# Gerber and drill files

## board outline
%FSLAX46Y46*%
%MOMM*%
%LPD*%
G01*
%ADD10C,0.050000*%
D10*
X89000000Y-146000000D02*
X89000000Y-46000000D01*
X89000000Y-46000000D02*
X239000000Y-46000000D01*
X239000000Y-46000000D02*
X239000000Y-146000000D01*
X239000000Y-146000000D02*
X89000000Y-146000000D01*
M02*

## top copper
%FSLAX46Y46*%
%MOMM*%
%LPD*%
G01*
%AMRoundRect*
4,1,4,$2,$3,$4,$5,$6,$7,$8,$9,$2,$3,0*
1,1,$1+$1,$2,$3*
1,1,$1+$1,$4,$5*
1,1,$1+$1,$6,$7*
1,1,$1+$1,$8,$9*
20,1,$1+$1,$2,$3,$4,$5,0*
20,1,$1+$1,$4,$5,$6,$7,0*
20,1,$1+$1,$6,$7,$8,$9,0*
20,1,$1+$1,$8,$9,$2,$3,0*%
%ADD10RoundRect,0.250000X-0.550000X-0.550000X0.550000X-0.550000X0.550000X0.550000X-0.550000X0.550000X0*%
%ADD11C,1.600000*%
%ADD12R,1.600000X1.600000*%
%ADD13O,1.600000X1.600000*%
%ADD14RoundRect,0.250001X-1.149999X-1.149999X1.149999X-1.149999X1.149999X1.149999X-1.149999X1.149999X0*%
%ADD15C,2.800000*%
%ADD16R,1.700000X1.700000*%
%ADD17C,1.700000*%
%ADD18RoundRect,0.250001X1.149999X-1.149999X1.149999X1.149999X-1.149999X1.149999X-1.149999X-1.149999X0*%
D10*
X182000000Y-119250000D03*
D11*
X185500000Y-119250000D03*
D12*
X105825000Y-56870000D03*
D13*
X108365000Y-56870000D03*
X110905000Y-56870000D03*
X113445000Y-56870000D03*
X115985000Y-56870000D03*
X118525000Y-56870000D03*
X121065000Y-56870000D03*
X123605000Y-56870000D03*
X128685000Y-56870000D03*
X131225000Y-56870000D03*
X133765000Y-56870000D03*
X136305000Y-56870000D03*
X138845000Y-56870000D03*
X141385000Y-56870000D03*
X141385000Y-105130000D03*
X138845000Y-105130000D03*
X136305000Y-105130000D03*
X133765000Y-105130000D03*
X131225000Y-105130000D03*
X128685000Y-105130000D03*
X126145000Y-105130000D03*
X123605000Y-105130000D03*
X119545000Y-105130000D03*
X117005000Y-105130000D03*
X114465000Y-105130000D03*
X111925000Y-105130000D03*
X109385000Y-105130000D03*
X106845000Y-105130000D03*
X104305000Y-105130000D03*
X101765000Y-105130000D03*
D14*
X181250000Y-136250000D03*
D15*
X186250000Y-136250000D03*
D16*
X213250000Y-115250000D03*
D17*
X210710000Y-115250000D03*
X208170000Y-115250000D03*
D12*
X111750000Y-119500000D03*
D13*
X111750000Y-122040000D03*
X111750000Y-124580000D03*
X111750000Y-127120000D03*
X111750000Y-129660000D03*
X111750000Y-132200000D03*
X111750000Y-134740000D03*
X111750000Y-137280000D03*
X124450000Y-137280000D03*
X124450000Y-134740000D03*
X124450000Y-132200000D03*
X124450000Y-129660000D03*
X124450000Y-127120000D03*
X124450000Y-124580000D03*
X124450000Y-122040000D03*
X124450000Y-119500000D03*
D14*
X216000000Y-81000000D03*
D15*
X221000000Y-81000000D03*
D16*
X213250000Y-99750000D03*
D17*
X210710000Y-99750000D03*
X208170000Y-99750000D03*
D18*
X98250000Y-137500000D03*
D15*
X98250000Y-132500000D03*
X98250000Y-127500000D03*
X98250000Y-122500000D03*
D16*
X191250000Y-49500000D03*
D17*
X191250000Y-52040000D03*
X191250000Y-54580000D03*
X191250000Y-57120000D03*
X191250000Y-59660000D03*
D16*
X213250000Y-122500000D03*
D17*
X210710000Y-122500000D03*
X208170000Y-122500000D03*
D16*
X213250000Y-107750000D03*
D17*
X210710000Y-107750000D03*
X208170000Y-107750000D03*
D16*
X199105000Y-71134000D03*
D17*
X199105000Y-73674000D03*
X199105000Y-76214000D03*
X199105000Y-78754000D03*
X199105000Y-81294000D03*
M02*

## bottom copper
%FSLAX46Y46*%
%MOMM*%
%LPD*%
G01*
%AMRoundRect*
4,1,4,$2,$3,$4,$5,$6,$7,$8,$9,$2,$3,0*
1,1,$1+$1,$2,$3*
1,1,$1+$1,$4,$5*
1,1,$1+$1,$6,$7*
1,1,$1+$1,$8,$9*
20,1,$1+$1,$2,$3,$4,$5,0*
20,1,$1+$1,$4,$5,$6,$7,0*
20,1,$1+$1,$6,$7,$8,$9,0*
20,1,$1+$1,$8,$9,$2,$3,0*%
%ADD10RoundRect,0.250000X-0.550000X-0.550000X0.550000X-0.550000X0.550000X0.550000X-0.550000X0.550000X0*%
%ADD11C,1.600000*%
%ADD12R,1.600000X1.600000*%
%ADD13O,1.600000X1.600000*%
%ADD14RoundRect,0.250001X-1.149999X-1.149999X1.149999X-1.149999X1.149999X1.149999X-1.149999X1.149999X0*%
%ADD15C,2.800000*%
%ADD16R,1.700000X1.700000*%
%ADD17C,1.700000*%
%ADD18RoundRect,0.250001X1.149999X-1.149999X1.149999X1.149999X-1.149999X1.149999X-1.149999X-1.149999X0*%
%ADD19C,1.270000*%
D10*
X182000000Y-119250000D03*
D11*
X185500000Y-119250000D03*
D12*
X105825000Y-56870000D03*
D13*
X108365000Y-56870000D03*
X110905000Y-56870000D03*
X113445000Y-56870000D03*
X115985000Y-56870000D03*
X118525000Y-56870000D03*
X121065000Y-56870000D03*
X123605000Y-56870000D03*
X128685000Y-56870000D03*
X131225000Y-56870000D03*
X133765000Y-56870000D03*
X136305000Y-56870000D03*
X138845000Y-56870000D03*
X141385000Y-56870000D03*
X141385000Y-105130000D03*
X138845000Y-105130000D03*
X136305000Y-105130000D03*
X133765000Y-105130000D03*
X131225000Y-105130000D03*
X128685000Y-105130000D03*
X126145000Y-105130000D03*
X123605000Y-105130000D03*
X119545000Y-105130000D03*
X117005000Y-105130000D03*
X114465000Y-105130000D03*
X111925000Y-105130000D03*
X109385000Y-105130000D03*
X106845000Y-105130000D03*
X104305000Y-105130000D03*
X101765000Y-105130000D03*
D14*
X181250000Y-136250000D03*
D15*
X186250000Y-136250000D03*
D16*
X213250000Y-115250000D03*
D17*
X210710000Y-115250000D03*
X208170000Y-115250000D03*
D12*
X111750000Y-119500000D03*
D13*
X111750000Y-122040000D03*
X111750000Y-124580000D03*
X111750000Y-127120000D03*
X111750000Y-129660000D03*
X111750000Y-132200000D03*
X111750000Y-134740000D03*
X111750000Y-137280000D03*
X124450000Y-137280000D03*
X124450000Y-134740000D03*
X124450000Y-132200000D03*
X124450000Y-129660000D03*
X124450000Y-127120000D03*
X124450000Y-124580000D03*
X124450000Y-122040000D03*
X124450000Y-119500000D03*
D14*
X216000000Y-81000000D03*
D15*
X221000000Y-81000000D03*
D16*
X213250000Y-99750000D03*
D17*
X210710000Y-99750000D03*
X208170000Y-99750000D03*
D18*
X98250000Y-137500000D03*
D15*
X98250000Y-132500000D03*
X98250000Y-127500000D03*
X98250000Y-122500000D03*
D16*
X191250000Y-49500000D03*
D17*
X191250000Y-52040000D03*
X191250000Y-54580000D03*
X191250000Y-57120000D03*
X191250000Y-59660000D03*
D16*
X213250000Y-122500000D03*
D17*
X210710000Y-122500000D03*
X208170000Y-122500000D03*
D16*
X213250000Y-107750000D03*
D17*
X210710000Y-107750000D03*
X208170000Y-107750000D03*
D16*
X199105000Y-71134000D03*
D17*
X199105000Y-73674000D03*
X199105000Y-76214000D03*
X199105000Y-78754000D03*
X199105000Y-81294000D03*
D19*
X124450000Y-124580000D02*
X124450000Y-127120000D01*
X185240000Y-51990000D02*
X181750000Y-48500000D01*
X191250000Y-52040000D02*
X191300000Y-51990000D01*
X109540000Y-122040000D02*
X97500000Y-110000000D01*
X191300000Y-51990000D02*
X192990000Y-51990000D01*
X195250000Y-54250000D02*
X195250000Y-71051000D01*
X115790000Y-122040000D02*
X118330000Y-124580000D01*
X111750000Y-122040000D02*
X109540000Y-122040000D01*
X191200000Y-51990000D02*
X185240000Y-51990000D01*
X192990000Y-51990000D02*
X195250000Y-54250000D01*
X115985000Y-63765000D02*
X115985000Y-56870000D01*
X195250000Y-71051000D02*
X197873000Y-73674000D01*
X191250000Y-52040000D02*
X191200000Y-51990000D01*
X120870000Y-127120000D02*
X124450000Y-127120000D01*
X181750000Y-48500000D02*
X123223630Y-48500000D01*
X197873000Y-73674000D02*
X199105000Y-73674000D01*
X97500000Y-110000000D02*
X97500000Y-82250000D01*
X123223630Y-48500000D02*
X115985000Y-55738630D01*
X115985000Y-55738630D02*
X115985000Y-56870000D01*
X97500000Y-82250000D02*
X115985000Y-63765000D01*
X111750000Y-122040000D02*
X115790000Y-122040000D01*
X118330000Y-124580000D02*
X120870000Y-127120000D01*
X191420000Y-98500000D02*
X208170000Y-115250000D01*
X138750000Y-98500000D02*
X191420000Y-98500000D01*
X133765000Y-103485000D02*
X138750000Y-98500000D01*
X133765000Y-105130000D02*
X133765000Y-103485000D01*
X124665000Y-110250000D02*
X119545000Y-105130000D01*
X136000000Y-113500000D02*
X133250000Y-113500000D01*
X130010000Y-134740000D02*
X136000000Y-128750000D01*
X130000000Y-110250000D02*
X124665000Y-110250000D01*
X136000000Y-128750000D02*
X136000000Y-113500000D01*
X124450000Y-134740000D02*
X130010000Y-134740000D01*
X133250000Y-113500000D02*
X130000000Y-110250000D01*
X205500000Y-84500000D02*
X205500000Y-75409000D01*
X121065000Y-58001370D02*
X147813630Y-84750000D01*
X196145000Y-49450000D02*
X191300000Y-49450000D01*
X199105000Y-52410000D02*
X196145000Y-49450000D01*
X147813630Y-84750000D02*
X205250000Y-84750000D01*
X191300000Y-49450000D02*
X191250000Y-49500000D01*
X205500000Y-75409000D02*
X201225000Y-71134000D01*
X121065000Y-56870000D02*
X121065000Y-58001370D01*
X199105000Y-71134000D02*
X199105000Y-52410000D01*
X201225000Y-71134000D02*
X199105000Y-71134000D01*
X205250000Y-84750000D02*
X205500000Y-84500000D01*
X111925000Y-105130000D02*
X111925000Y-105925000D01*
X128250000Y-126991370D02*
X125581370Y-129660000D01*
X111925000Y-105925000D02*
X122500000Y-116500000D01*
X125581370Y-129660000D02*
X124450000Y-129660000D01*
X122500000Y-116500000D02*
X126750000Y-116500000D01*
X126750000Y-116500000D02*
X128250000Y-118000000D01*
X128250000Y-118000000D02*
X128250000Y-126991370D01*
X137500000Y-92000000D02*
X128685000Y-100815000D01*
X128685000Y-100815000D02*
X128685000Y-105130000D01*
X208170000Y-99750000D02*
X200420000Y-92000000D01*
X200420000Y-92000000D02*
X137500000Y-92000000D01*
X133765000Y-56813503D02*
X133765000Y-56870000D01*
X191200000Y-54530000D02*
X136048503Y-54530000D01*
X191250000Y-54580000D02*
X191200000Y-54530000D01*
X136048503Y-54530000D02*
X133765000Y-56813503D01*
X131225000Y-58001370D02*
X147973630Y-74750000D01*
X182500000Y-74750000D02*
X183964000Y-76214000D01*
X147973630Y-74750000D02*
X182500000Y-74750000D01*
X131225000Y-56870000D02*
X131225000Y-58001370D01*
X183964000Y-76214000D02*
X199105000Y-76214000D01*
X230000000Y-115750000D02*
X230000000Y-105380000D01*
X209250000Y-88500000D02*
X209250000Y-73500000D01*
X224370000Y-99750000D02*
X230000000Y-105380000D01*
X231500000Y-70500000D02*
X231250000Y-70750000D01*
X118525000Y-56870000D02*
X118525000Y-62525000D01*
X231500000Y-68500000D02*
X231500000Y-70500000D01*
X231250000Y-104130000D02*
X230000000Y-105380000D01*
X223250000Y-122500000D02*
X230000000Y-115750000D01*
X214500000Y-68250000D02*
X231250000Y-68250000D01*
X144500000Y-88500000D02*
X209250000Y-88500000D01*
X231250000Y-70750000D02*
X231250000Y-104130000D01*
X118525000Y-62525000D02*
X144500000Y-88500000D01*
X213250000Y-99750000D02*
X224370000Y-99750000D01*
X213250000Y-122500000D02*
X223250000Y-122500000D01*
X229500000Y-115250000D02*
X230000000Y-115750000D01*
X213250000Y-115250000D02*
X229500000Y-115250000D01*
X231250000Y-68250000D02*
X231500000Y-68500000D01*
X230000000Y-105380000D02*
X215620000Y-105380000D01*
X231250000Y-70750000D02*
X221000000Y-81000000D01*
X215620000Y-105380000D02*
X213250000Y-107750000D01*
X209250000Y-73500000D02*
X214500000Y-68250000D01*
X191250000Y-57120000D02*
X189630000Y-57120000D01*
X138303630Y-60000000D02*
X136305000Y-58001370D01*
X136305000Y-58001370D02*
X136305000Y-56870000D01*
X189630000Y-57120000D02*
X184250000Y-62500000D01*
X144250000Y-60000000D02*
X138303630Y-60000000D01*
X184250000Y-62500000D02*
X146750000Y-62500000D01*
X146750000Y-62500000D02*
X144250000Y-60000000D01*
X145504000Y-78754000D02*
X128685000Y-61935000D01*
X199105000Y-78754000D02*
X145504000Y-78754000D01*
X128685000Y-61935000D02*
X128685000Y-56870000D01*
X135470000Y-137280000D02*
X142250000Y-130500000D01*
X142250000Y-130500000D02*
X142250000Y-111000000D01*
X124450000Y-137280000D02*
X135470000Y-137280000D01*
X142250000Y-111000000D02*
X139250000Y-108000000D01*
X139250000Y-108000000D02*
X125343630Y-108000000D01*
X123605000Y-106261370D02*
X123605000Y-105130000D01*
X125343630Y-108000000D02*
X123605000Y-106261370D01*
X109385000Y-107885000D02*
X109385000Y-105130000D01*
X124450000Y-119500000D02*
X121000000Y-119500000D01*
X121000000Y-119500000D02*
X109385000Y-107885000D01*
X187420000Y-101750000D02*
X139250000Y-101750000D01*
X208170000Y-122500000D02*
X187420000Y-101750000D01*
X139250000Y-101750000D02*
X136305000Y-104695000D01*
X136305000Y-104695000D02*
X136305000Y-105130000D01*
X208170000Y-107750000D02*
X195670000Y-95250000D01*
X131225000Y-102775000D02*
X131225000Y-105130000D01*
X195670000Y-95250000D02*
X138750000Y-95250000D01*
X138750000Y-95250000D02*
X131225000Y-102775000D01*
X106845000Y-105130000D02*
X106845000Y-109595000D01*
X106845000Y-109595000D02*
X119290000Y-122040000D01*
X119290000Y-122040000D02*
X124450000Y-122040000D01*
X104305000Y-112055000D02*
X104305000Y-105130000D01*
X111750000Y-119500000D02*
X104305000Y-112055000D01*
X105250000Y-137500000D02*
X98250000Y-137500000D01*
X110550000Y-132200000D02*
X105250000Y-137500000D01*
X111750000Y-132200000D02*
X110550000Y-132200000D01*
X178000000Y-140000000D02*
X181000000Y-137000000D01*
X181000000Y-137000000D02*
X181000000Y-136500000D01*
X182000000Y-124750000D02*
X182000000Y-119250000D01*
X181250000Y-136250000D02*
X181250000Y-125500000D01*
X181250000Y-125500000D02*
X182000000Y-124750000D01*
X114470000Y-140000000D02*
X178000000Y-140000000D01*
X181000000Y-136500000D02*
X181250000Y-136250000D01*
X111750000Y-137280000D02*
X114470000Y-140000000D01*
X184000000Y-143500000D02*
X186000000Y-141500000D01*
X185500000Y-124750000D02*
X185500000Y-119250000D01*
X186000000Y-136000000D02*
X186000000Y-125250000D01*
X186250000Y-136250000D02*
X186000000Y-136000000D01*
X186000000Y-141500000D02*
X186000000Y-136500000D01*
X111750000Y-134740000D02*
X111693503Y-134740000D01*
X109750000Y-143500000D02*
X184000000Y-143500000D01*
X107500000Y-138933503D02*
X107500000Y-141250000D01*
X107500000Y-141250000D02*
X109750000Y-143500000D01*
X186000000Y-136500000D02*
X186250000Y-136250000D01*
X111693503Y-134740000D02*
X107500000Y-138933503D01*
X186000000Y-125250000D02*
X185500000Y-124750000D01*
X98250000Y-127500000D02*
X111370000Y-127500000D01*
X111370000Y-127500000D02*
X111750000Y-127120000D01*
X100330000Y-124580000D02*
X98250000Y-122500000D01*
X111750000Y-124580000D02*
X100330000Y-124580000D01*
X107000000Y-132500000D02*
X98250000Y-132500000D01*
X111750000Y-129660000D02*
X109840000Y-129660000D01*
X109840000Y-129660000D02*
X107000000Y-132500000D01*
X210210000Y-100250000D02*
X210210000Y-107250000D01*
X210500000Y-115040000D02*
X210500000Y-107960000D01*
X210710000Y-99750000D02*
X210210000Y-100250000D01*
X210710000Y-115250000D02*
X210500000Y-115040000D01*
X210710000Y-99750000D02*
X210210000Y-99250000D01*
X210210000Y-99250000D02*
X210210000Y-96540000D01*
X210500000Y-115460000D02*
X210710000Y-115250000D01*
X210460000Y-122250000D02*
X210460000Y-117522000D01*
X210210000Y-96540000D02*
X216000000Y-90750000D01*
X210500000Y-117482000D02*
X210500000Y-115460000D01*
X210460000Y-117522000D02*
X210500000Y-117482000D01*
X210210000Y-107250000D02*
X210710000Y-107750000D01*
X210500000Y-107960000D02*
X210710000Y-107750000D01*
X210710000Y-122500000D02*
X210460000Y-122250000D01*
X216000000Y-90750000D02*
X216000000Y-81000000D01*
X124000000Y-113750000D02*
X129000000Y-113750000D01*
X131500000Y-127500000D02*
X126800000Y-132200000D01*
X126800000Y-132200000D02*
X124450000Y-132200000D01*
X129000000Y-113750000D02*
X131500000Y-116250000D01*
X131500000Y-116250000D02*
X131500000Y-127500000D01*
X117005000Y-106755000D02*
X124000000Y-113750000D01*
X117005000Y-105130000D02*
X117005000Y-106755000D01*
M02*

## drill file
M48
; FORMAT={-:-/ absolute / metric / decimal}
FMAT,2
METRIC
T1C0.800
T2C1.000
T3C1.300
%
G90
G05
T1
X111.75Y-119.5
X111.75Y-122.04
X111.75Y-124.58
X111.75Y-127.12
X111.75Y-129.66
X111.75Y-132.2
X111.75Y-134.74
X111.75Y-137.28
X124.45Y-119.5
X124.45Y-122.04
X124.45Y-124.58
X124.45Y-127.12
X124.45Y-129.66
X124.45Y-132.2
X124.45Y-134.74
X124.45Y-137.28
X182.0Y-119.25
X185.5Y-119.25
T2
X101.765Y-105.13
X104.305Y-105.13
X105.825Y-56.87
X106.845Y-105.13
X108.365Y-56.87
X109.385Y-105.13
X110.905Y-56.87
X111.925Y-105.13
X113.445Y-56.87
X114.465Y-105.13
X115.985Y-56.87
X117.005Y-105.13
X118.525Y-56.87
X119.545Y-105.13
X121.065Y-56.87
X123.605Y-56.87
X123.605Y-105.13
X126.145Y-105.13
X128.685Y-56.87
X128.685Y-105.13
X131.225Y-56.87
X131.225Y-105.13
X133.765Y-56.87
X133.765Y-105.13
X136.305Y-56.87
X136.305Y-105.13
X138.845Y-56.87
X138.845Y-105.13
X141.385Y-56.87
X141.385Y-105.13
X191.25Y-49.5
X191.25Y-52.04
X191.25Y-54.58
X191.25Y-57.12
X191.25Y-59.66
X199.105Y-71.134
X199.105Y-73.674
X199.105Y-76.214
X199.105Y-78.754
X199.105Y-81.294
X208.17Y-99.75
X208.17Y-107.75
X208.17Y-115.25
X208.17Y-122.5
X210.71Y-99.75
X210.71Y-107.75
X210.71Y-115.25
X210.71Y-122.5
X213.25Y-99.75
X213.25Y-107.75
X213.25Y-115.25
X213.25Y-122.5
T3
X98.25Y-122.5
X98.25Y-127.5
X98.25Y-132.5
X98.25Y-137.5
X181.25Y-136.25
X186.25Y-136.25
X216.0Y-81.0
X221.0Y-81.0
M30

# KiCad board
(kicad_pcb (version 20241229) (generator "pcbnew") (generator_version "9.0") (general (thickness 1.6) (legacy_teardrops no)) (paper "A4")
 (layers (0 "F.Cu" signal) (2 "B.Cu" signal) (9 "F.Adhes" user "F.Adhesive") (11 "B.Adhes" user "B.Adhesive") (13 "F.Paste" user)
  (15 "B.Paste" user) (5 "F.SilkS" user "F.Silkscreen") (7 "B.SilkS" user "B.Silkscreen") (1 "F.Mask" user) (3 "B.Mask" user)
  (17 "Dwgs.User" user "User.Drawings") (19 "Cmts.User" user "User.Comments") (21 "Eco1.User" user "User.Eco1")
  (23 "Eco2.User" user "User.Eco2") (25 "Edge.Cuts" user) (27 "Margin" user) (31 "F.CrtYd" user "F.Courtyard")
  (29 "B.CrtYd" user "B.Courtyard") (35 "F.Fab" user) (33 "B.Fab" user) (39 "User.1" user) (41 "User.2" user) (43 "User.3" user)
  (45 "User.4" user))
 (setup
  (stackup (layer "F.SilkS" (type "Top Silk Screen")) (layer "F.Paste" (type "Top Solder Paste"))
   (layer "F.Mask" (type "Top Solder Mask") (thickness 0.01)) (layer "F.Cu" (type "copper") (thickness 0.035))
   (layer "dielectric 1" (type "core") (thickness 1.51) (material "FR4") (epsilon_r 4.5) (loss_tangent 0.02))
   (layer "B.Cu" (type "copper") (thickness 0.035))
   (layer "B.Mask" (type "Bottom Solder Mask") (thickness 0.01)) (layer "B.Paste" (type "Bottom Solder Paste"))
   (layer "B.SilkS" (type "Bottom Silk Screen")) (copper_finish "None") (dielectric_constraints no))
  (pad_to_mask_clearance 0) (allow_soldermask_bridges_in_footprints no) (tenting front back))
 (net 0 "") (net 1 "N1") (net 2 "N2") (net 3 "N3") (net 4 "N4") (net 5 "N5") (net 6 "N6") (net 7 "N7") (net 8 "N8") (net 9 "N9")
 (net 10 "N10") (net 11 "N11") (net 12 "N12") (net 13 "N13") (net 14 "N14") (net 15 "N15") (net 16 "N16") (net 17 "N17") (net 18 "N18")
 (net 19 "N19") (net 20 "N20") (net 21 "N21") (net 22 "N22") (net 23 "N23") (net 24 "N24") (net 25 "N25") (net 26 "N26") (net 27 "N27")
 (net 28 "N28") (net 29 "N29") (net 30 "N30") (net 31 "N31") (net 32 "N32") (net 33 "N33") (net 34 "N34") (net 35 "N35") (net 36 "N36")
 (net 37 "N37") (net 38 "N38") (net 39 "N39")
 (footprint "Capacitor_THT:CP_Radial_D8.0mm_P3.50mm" (layer "F.Cu") (at 182 119.25)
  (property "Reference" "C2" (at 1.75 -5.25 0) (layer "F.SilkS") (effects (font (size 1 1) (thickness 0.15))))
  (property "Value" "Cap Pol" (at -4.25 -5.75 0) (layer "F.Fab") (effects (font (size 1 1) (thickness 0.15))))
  (pad "1" thru_hole roundrect (at 0 0) (size 1.6 1.6) (drill 0.8) (layers "*.Cu" "*.Mask") (remove_unused_layers no)
   (roundrect_rratio 0.15625) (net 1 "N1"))
  (pad "2" thru_hole circle (at 3.5 0) (size 1.6 1.6) (drill 0.8) (layers "*.Cu" "*.Mask") (remove_unused_layers no) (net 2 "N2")))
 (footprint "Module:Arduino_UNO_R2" (layer "F.Cu") (at 105.825 56.87)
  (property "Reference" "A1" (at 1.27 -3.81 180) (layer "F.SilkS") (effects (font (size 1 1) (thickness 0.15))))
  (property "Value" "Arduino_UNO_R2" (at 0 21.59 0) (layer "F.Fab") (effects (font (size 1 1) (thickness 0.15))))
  (pad "1" thru_hole rect (at 0 0 90) (size 1.6 1.6) (drill 1) (layers "*.Cu" "*.Mask") (remove_unused_layers no) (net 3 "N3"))
  (pad "2" thru_hole oval (at 2.54 0 90) (size 1.6 1.6) (drill 1) (layers "*.Cu" "*.Mask") (remove_unused_layers no) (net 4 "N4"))
  (pad "3" thru_hole oval (at 5.08 0 90) (size 1.6 1.6) (drill 1) (layers "*.Cu" "*.Mask") (remove_unused_layers no) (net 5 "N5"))
  (pad "4" thru_hole oval (at 7.62 0 90) (size 1.6 1.6) (drill 1) (layers "*.Cu" "*.Mask") (remove_unused_layers no) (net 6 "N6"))
  (pad "5" thru_hole oval (at 10.16 0 90) (size 1.6 1.6) (drill 1) (layers "*.Cu" "*.Mask") (remove_unused_layers no) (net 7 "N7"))
  (pad "6" thru_hole oval (at 12.7 0 90) (size 1.6 1.6) (drill 1) (layers "*.Cu" "*.Mask") (remove_unused_layers no) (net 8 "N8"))
  (pad "7" thru_hole oval (at 15.24 0 90) (size 1.6 1.6) (drill 1) (layers "*.Cu" "*.Mask") (remove_unused_layers no) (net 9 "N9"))
  (pad "8" thru_hole oval (at 17.78 0 90) (size 1.6 1.6) (drill 1) (layers "*.Cu" "*.Mask") (remove_unused_layers no) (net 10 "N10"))
  (pad "9" thru_hole oval (at 22.86 0 90) (size 1.6 1.6) (drill 1) (layers "*.Cu" "*.Mask") (remove_unused_layers no) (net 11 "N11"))
  (pad "10" thru_hole oval (at 25.4 0 90) (size 1.6 1.6) (drill 1) (layers "*.Cu" "*.Mask") (remove_unused_layers no) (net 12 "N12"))
  (pad "11" thru_hole oval (at 27.94 0 90) (size 1.6 1.6) (drill 1) (layers "*.Cu" "*.Mask") (remove_unused_layers no) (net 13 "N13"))
  (pad "12" thru_hole oval (at 30.48 0 90) (size 1.6 1.6) (drill 1) (layers "*.Cu" "*.Mask") (remove_unused_layers no) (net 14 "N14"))
  (pad "13" thru_hole oval (at 33.02 0 90) (size 1.6 1.6) (drill 1) (layers "*.Cu" "*.Mask") (remove_unused_layers no) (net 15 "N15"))
  (pad "14" thru_hole oval (at 35.56 0 90) (size 1.6 1.6) (drill 1) (layers "*.Cu" "*.Mask") (remove_unused_layers no) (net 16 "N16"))
  (pad "15" thru_hole oval (at 35.56 48.26 90) (size 1.6 1.6) (drill 1) (layers "*.Cu" "*.Mask") (remove_unused_layers no) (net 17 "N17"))
  (pad "16" thru_hole oval (at 33.02 48.26 90) (size 1.6 1.6) (drill 1) (layers "*.Cu" "*.Mask") (remove_unused_layers no) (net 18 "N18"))
  (pad "17" thru_hole oval (at 30.48 48.26 90) (size 1.6 1.6) (drill 1) (layers "*.Cu" "*.Mask") (remove_unused_layers no) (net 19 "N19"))
  (pad "18" thru_hole oval (at 27.94 48.26 90) (size 1.6 1.6) (drill 1) (layers "*.Cu" "*.Mask") (remove_unused_layers no) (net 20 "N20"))
  (pad "19" thru_hole oval (at 25.4 48.26 90) (size 1.6 1.6) (drill 1) (layers "*.Cu" "*.Mask") (remove_unused_layers no) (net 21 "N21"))
  (pad "20" thru_hole oval (at 22.86 48.26 90) (size 1.6 1.6) (drill 1) (layers "*.Cu" "*.Mask") (remove_unused_layers no) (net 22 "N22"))
  (pad "21" thru_hole oval (at 20.32 48.26 90) (size 1.6 1.6) (drill 1) (layers "*.Cu" "*.Mask") (remove_unused_layers no) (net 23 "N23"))
  (pad "22" thru_hole oval (at 17.78 48.26 90) (size 1.6 1.6) (drill 1) (layers "*.Cu" "*.Mask") (remove_unused_layers no) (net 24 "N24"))
  (pad "23" thru_hole oval (at 13.72 48.26 90) (size 1.6 1.6) (drill 1) (layers "*.Cu" "*.Mask") (remove_unused_layers no) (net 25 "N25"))
  (pad "24" thru_hole oval (at 11.18 48.26 90) (size 1.6 1.6) (drill 1) (layers "*.Cu" "*.Mask") (remove_unused_layers no) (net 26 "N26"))
  (pad "25" thru_hole oval (at 8.64 48.26 90) (size 1.6 1.6) (drill 1) (layers "*.Cu" "*.Mask") (remove_unused_layers no) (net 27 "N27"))
  (pad "26" thru_hole oval (at 6.1 48.26 90) (size 1.6 1.6) (drill 1) (layers "*.Cu" "*.Mask") (remove_unused_layers no) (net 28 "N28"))
  (pad "27" thru_hole oval (at 3.56 48.26 90) (size 1.6 1.6) (drill 1) (layers "*.Cu" "*.Mask") (remove_unused_layers no) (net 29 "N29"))
  (pad "28" thru_hole oval (at 1.02 48.26 90) (size 1.6 1.6) (drill 1) (layers "*.Cu" "*.Mask") (remove_unused_layers no) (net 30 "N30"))
  (pad "29" thru_hole oval (at -1.52 48.26 90) (size 1.6 1.6) (drill 1) (layers "*.Cu" "*.Mask") (remove_unused_layers no) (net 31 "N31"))
  (pad "30" thru_hole oval (at -4.06 48.26 90) (size 1.6 1.6) (drill 1) (layers "*.Cu" "*.Mask") (remove_unused_layers no) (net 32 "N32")))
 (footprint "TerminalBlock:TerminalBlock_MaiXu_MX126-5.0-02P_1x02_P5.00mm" (layer "F.Cu") (at 181.25 136.25)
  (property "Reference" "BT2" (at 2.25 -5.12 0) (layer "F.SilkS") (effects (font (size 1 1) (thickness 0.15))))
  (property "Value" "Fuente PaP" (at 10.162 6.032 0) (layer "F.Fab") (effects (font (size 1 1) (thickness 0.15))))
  (pad "1" thru_hole roundrect (at 0 0) (size 2.8 2.8) (drill 1.3) (layers "*.Cu" "*.Mask") (remove_unused_layers no)
   (roundrect_rratio 0.089286) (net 1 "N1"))
  (pad "2" thru_hole circle (at 5 0) (size 2.8 2.8) (drill 1.3) (layers "*.Cu" "*.Mask") (remove_unused_layers no) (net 2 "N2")))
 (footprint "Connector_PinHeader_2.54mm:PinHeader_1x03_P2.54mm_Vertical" (layer "F.Cu") (at 213.25 115.25 -90)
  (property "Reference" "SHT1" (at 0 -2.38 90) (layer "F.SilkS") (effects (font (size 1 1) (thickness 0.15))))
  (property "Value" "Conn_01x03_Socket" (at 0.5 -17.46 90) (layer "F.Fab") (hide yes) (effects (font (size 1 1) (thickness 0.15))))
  (pad "1" thru_hole rect (at 0 0 270) (size 1.7 1.7) (drill 1) (layers "*.Cu" "*.Mask") (remove_unused_layers no) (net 8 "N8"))
  (pad "2" thru_hole circle (at 0 2.54 270) (size 1.7 1.7) (drill 1) (layers "*.Cu" "*.Mask") (remove_unused_layers no) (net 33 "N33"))
  (pad "3" thru_hole circle (at 0 5.08 270) (size 1.7 1.7) (drill 1) (layers "*.Cu" "*.Mask") (remove_unused_layers no) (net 20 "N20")))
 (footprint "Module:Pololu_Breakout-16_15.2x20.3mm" (layer "F.Cu") (at 111.75 119.5)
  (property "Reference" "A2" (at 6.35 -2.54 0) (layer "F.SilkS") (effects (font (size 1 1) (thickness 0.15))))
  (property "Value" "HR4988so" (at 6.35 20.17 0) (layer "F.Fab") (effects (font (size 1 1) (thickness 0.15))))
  (pad "1" thru_hole rect (at 0 0) (size 1.6 1.6) (drill 0.8) (layers "*.Cu" "*.Mask") (remove_unused_layers no) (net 31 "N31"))
  (pad "2" thru_hole oval (at 0 2.54) (size 1.6 1.6) (drill 0.8) (layers "*.Cu" "*.Mask") (remove_unused_layers no) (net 7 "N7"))
  (pad "3" thru_hole oval (at 0 5.08) (size 1.6 1.6) (drill 0.8) (layers "*.Cu" "*.Mask") (remove_unused_layers no) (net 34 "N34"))
  (pad "4" thru_hole oval (at 0 7.62) (size 1.6 1.6) (drill 0.8) (layers "*.Cu" "*.Mask") (remove_unused_layers no) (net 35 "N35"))
  (pad "5" thru_hole oval (at 0 10.16) (size 1.6 1.6) (drill 0.8) (layers "*.Cu" "*.Mask") (remove_unused_layers no) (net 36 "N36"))
  (pad "6" thru_hole oval (at 0 12.7) (size 1.6 1.6) (drill 0.8) (layers "*.Cu" "*.Mask") (remove_unused_layers no) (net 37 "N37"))
  (pad "7" thru_hole oval (at 0 15.24) (size 1.6 1.6) (drill 0.8) (layers "*.Cu" "*.Mask") (remove_unused_layers no) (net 2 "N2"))
  (pad "8" thru_hole oval (at 0 17.78) (size 1.6 1.6) (drill 0.8) (layers "*.Cu" "*.Mask") (remove_unused_layers no) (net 1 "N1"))
  (pad "9" thru_hole oval (at 12.7 17.78) (size 1.6 1.6) (drill 0.8) (layers "*.Cu" "*.Mask") (remove_unused_layers no) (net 24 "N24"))
  (pad "10" thru_hole oval (at 12.7 15.24) (size 1.6 1.6) (drill 0.8) (layers "*.Cu" "*.Mask") (remove_unused_layers no) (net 25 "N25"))
  (pad "11" thru_hole oval (at 12.7 12.7) (size 1.6 1.6) (drill 0.8) (layers "*.Cu" "*.Mask") (remove_unused_layers no) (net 26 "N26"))
  (pad "12" thru_hole oval (at 12.7 10.16) (size 1.6 1.6) (drill 0.8) (layers "*.Cu" "*.Mask") (remove_unused_layers no) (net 28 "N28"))
  (pad "13" thru_hole oval (at 12.7 7.62) (size 1.6 1.6) (drill 0.8) (layers "*.Cu" "*.Mask") (remove_unused_layers no) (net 7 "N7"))
  (pad "14" thru_hole oval (at 12.7 5.08) (size 1.6 1.6) (drill 0.8) (layers "*.Cu" "*.Mask") (remove_unused_layers no) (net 7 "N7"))
  (pad "15" thru_hole oval (at 12.7 2.54) (size 1.6 1.6) (drill 0.8) (layers "*.Cu" "*.Mask") (remove_unused_layers no) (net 30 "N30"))
  (pad "16" thru_hole oval (at 12.7 0) (size 1.6 1.6) (drill 0.8) (layers "*.Cu" "*.Mask") (remove_unused_layers no) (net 29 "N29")))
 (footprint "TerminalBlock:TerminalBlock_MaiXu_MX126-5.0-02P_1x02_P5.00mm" (layer "F.Cu") (at 216 81)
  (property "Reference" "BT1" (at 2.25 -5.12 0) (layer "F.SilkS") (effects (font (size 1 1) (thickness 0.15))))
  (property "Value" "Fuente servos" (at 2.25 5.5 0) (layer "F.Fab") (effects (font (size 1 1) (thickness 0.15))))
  (pad "1" thru_hole roundrect (at 0 0) (size 2.8 2.8) (drill 1.3) (layers "*.Cu" "*.Mask") (remove_unused_layers no)
   (roundrect_rratio 0.089286) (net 33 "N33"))
  (pad "2" thru_hole circle (at 5 0) (size 2.8 2.8) (drill 1.3) (layers "*.Cu" "*.Mask") (remove_unused_layers no) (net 8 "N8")))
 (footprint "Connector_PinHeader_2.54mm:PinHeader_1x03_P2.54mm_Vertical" (layer "F.Cu") (at 213.25 99.75 -90)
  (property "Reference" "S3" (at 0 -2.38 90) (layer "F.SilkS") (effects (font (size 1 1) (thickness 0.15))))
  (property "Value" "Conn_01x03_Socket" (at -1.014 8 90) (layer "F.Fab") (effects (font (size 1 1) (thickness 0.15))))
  (pad "1" thru_hole rect (at 0 0 270) (size 1.7 1.7) (drill 1) (layers "*.Cu" "*.Mask") (remove_unused_layers no) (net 8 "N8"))
  (pad "2" thru_hole circle (at 0 2.54 270) (size 1.7 1.7) (drill 1) (layers "*.Cu" "*.Mask") (remove_unused_layers no) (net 33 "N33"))
  (pad "3" thru_hole circle (at 0 5.08 270) (size 1.7 1.7) (drill 1) (layers "*.Cu" "*.Mask") (remove_unused_layers no) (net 22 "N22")))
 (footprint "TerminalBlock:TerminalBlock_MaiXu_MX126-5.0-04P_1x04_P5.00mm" (layer "F.Cu") (at 98.25 137.5 90)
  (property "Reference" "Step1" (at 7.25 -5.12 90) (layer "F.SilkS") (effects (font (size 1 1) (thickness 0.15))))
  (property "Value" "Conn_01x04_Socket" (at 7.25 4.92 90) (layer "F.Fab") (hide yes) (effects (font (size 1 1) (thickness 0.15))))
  (pad "1" thru_hole roundrect (at 0 0 90) (size 2.8 2.8) (drill 1.3) (layers "*.Cu" "*.Mask") (remove_unused_layers no)
   (roundrect_rratio 0.089286) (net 37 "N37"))
  (pad "2" thru_hole circle (at 5 0 90) (size 2.8 2.8) (drill 1.3) (layers "*.Cu" "*.Mask") (remove_unused_layers no) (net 36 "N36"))
  (pad "3" thru_hole circle (at 10 0 90) (size 2.8 2.8) (drill 1.3) (layers "*.Cu" "*.Mask") (remove_unused_layers no) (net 35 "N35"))
  (pad "4" thru_hole circle (at 15 0 90) (size 2.8 2.8) (drill 1.3) (layers "*.Cu" "*.Mask") (remove_unused_layers no) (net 34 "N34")))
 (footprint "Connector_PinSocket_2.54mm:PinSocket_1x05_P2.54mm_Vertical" (layer "F.Cu") (at 191.25 49.5)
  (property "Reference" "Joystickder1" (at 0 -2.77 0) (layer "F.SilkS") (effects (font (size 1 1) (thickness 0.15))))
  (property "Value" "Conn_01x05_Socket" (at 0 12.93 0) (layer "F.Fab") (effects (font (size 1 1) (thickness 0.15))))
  (pad "1" thru_hole rect (at 0 0) (size 1.7 1.7) (drill 1) (layers "*.Cu" "*.Mask") (remove_unused_layers no) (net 9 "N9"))
  (pad "2" thru_hole circle (at 0 2.54) (size 1.7 1.7) (drill 1) (layers "*.Cu" "*.Mask") (remove_unused_layers no) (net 7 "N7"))
  (pad "3" thru_hole circle (at 0 5.08) (size 1.7 1.7) (drill 1) (layers "*.Cu" "*.Mask") (remove_unused_layers no) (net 13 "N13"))
  (pad "4" thru_hole circle (at 0 7.62) (size 1.7 1.7) (drill 1) (layers "*.Cu" "*.Mask") (remove_unused_layers no) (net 14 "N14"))
  (pad "5" thru_hole circle (at 0 10.16) (size 1.7 1.7) (drill 1) (layers "*.Cu" "*.Mask") (remove_unused_layers no) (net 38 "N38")))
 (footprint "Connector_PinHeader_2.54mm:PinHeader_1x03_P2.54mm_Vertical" (layer "F.Cu") (at 213.25 122.5 -90)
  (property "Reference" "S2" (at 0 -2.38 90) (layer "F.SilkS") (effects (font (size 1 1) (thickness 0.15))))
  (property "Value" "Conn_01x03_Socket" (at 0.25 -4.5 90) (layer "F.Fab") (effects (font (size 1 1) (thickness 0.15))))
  (pad "1" thru_hole rect (at 0 0 270) (size 1.7 1.7) (drill 1) (layers "*.Cu" "*.Mask") (remove_unused_layers no) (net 8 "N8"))
  (pad "2" thru_hole circle (at 0 2.54 270) (size 1.7 1.7) (drill 1) (layers "*.Cu" "*.Mask") (remove_unused_layers no) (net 33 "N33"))
  (pad "3" thru_hole circle (at 0 5.08 270) (size 1.7 1.7) (drill 1) (layers "*.Cu" "*.Mask") (remove_unused_layers no) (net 19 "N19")))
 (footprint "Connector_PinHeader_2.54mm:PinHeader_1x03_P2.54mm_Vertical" (layer "F.Cu") (at 213.25 107.75 -90)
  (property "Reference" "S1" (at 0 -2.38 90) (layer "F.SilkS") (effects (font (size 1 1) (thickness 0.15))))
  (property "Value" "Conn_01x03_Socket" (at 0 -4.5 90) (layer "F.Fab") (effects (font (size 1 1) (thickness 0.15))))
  (pad "1" thru_hole rect (at 0 0 270) (size 1.7 1.7) (drill 1) (layers "*.Cu" "*.Mask") (remove_unused_layers no) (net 8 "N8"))
  (pad "2" thru_hole circle (at 0 2.54 270) (size 1.7 1.7) (drill 1) (layers "*.Cu" "*.Mask") (remove_unused_layers no) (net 33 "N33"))
  (pad "3" thru_hole circle (at 0 5.08 270) (size 1.7 1.7) (drill 1) (layers "*.Cu" "*.Mask") (remove_unused_layers no) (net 21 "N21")))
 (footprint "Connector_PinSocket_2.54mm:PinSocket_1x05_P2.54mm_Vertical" (layer "F.Cu") (at 199.105 71.134)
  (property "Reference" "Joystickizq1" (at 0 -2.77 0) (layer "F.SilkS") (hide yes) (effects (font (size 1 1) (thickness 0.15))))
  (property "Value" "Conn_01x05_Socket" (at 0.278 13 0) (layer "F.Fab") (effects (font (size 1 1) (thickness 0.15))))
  (pad "1" thru_hole rect (at 0 0) (size 1.7 1.7) (drill 1) (layers "*.Cu" "*.Mask") (remove_unused_layers no) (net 9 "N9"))
  (pad "2" thru_hole circle (at 0 2.54) (size 1.7 1.7) (drill 1) (layers "*.Cu" "*.Mask") (remove_unused_layers no) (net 7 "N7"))
  (pad "3" thru_hole circle (at 0 5.08) (size 1.7 1.7) (drill 1) (layers "*.Cu" "*.Mask") (remove_unused_layers no) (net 12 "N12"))
  (pad "4" thru_hole circle (at 0 7.62) (size 1.7 1.7) (drill 1) (layers "*.Cu" "*.Mask") (remove_unused_layers no) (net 11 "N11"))
  (pad "5" thru_hole circle (at 0 10.16) (size 1.7 1.7) (drill 1) (layers "*.Cu" "*.Mask") (remove_unused_layers no) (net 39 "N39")))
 (gr_line (start 89 146) (end 89 46) (stroke (width 0.05) (type default)) (layer "Edge.Cuts"))
 (gr_line (start 89 46) (end 239 46) (stroke (width 0.05) (type default)) (layer "Edge.Cuts"))
 (gr_line (start 239 46) (end 239 146) (stroke (width 0.05) (type default)) (layer "Edge.Cuts"))
 (gr_line (start 239 146) (end 89 146) (stroke (width 0.05) (type default)) (layer "Edge.Cuts"))
 (segment (start 124.45 124.58) (end 124.45 127.12) (width 1.27) (layer "B.Cu") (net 7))
 (segment (start 185.24 51.99) (end 181.75 48.5) (width 1.27) (layer "B.Cu") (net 7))
 (segment (start 191.25 52.04) (end 191.3 51.99) (width 1.27) (layer "B.Cu") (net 7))
 (segment (start 109.54 122.04) (end 97.5 110) (width 1.27) (layer "B.Cu") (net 7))
 (segment (start 191.3 51.99) (end 192.99 51.99) (width 1.27) (layer "B.Cu") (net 7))
 (segment (start 195.25 54.25) (end 195.25 71.051) (width 1.27) (layer "B.Cu") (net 7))
 (segment (start 115.79 122.04) (end 118.33 124.58) (width 1.27) (layer "B.Cu") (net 7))
 (segment (start 111.75 122.04) (end 109.54 122.04) (width 1.27) (layer "B.Cu") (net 7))
 (segment (start 191.2 51.99) (end 185.24 51.99) (width 1.27) (layer "B.Cu") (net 7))
 (segment (start 192.99 51.99) (end 195.25 54.25) (width 1.27) (layer "B.Cu") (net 7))
 (segment (start 115.985 63.765) (end 115.985 56.87) (width 1.27) (layer "B.Cu") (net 7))
 (segment (start 195.25 71.051) (end 197.873 73.674) (width 1.27) (layer "B.Cu") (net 7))
 (segment (start 191.25 52.04) (end 191.2 51.99) (width 1.27) (layer "B.Cu") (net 7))
 (segment (start 120.87 127.12) (end 124.45 127.12) (width 1.27) (layer "B.Cu") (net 7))
 (segment (start 181.75 48.5) (end 123.22363 48.5) (width 1.27) (layer "B.Cu") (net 7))
 (segment (start 197.873 73.674) (end 199.105 73.674) (width 1.27) (layer "B.Cu") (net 7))
 (segment (start 97.5 110) (end 97.5 82.25) (width 1.27) (layer "B.Cu") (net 7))
 (segment (start 123.22363 48.5) (end 115.985 55.73863) (width 1.27) (layer "B.Cu") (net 7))
 (segment (start 115.985 55.73863) (end 115.985 56.87) (width 1.27) (layer "B.Cu") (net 7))
 (segment (start 97.5 82.25) (end 115.985 63.765) (width 1.27) (layer "B.Cu") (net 7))
 (segment (start 111.75 122.04) (end 115.79 122.04) (width 1.27) (layer "B.Cu") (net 7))
 (segment (start 118.33 124.58) (end 120.87 127.12) (width 1.27) (layer "B.Cu") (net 7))
 (segment (start 191.42 98.5) (end 208.17 115.25) (width 1.27) (layer "B.Cu") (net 20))
 (segment (start 138.75 98.5) (end 191.42 98.5) (width 1.27) (layer "B.Cu") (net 20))
 (segment (start 133.765 103.485) (end 138.75 98.5) (width 1.27) (layer "B.Cu") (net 20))
 (segment (start 133.765 105.13) (end 133.765 103.485) (width 1.27) (layer "B.Cu") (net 20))
 (segment (start 124.665 110.25) (end 119.545 105.13) (width 1.27) (layer "B.Cu") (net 25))
 (segment (start 136 113.5) (end 133.25 113.5) (width 1.27) (layer "B.Cu") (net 25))
 (segment (start 130.01 134.74) (end 136 128.75) (width 1.27) (layer "B.Cu") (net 25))
 (segment (start 130 110.25) (end 124.665 110.25) (width 1.27) (layer "B.Cu") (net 25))
 (segment (start 136 128.75) (end 136 113.5) (width 1.27) (layer "B.Cu") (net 25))
 (segment (start 124.45 134.74) (end 130.01 134.74) (width 1.27) (layer "B.Cu") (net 25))
 (segment (start 133.25 113.5) (end 130 110.25) (width 1.27) (layer "B.Cu") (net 25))
 (segment (start 205.5 84.5) (end 205.5 75.409) (width 1.27) (layer "B.Cu") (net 9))
 (segment (start 121.065 58.00137) (end 147.81363 84.75) (width 1.27) (layer "B.Cu") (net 9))
 (segment (start 196.145 49.45) (end 191.3 49.45) (width 1.27) (layer "B.Cu") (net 9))
 (segment (start 199.105 52.41) (end 196.145 49.45) (width 1.27) (layer "B.Cu") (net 9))
 (segment (start 147.81363 84.75) (end 205.25 84.75) (width 1.27) (layer "B.Cu") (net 9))
 (segment (start 191.3 49.45) (end 191.25 49.5) (width 1.27) (layer "B.Cu") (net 9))
 (segment (start 205.5 75.409) (end 201.225 71.134) (width 1.27) (layer "B.Cu") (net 9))
 (segment (start 121.065 56.87) (end 121.065 58.00137) (width 1.27) (layer "B.Cu") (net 9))
 (segment (start 199.105 71.134) (end 199.105 52.41) (width 1.27) (layer "B.Cu") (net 9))
 (segment (start 201.225 71.134) (end 199.105 71.134) (width 1.27) (layer "B.Cu") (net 9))
 (segment (start 205.25 84.75) (end 205.5 84.5) (width 1.27) (layer "B.Cu") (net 9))
 (segment (start 111.925 105.13) (end 111.925 105.925) (width 1.27) (layer "B.Cu") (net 28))
 (segment (start 128.25 126.99137) (end 125.58137 129.66) (width 1.27) (layer "B.Cu") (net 28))
 (segment (start 111.925 105.925) (end 122.5 116.5) (width 1.27) (layer "B.Cu") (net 28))
 (segment (start 125.58137 129.66) (end 124.45 129.66) (width 1.27) (layer "B.Cu") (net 28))
 (segment (start 122.5 116.5) (end 126.75 116.5) (width 1.27) (layer "B.Cu") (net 28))
 (segment (start 126.75 116.5) (end 128.25 118) (width 1.27) (layer "B.Cu") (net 28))
 (segment (start 128.25 118) (end 128.25 126.99137) (width 1.27) (layer "B.Cu") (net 28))
 (segment (start 137.5 92) (end 128.685 100.815) (width 1.27) (layer "B.Cu") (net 22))
 (segment (start 128.685 100.815) (end 128.685 105.13) (width 1.27) (layer "B.Cu") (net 22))
 (segment (start 208.17 99.75) (end 200.42 92) (width 1.27) (layer "B.Cu") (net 22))
 (segment (start 200.42 92) (end 137.5 92) (width 1.27) (layer "B.Cu") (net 22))
 (segment (start 133.765 56.813503) (end 133.765 56.87) (width 1.27) (layer "B.Cu") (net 13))
 (segment (start 191.2 54.53) (end 136.048503 54.53) (width 1.27) (layer "B.Cu") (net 13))
 (segment (start 191.25 54.58) (end 191.2 54.53) (width 1.27) (layer "B.Cu") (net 13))
 (segment (start 136.048503 54.53) (end 133.765 56.813503) (width 1.27) (layer "B.Cu") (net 13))
 (segment (start 131.225 58.00137) (end 147.97363 74.75) (width 1.27) (layer "B.Cu") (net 12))
 (segment (start 182.5 74.75) (end 183.964 76.214) (width 1.27) (layer "B.Cu") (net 12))
 (segment (start 147.97363 74.75) (end 182.5 74.75) (width 1.27) (layer "B.Cu") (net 12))
 (segment (start 131.225 56.87) (end 131.225 58.00137) (width 1.27) (layer "B.Cu") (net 12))
 (segment (start 183.964 76.214) (end 199.105 76.214) (width 1.27) (layer "B.Cu") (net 12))
 (segment (start 230 115.75) (end 230 105.38) (width 1.27) (layer "B.Cu") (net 8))
 (segment (start 209.25 88.5) (end 209.25 73.5) (width 1.27) (layer "B.Cu") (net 8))
 (segment (start 224.37 99.75) (end 230 105.38) (width 1.27) (layer "B.Cu") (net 8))
 (segment (start 231.5 70.5) (end 231.25 70.75) (width 1.27) (layer "B.Cu") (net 8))
 (segment (start 118.525 56.87) (end 118.525 62.525) (width 1.27) (layer "B.Cu") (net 8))
 (segment (start 231.5 68.5) (end 231.5 70.5) (width 1.27) (layer "B.Cu") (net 8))
 (segment (start 231.25 104.13) (end 230 105.38) (width 1.27) (layer "B.Cu") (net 8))
 (segment (start 223.25 122.5) (end 230 115.75) (width 1.27) (layer "B.Cu") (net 8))
 (segment (start 214.5 68.25) (end 231.25 68.25) (width 1.27) (layer "B.Cu") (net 8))
 (segment (start 144.5 88.5) (end 209.25 88.5) (width 1.27) (layer "B.Cu") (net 8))
 (segment (start 231.25 70.75) (end 231.25 104.13) (width 1.27) (layer "B.Cu") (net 8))
 (segment (start 118.525 62.525) (end 144.5 88.5) (width 1.27) (layer "B.Cu") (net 8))
 (segment (start 213.25 99.75) (end 224.37 99.75) (width 1.27) (layer "B.Cu") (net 8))
 (segment (start 213.25 122.5) (end 223.25 122.5) (width 1.27) (layer "B.Cu") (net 8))
 (segment (start 229.5 115.25) (end 230 115.75) (width 1.27) (layer "B.Cu") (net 8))
 (segment (start 213.25 115.25) (end 229.5 115.25) (width 1.27) (layer "B.Cu") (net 8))
 (segment (start 231.25 68.25) (end 231.5 68.5) (width 1.27) (layer "B.Cu") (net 8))
 (segment (start 230 105.38) (end 215.62 105.38) (width 1.27) (layer "B.Cu") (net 8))
 (segment (start 231.25 70.75) (end 221 81) (width 1.27) (layer "B.Cu") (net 8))
 (segment (start 215.62 105.38) (end 213.25 107.75) (width 1.27) (layer "B.Cu") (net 8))
 (segment (start 209.25 73.5) (end 214.5 68.25) (width 1.27) (layer "B.Cu") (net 8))
 (segment (start 191.25 57.12) (end 189.63 57.12) (width 1.27) (layer "B.Cu") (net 14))
 (segment (start 138.30363 60) (end 136.305 58.00137) (width 1.27) (layer "B.Cu") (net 14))
 (segment (start 136.305 58.00137) (end 136.305 56.87) (width 1.27) (layer "B.Cu") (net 14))
 (segment (start 189.63 57.12) (end 184.25 62.5) (width 1.27) (layer "B.Cu") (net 14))
 (segment (start 144.25 60) (end 138.30363 60) (width 1.27) (layer "B.Cu") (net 14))
 (segment (start 184.25 62.5) (end 146.75 62.5) (width 1.27) (layer "B.Cu") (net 14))
 (segment (start 146.75 62.5) (end 144.25 60) (width 1.27) (layer "B.Cu") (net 14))
 (segment (start 145.504 78.754) (end 128.685 61.935) (width 1.27) (layer "B.Cu") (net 11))
 (segment (start 199.105 78.754) (end 145.504 78.754) (width 1.27) (layer "B.Cu") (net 11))
 (segment (start 128.685 61.935) (end 128.685 56.87) (width 1.27) (layer "B.Cu") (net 11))
 (segment (start 135.47 137.28) (end 142.25 130.5) (width 1.27) (layer "B.Cu") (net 24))
 (segment (start 142.25 130.5) (end 142.25 111) (width 1.27) (layer "B.Cu") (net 24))
 (segment (start 124.45 137.28) (end 135.47 137.28) (width 1.27) (layer "B.Cu") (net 24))
 (segment (start 142.25 111) (end 139.25 108) (width 1.27) (layer "B.Cu") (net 24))
 (segment (start 139.25 108) (end 125.34363 108) (width 1.27) (layer "B.Cu") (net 24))
 (segment (start 123.605 106.26137) (end 123.605 105.13) (width 1.27) (layer "B.Cu") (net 24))
 (segment (start 125.34363 108) (end 123.605 106.26137) (width 1.27) (layer "B.Cu") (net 24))
 (segment (start 109.385 107.885) (end 109.385 105.13) (width 1.27) (layer "B.Cu") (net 29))
 (segment (start 124.45 119.5) (end 121 119.5) (width 1.27) (layer "B.Cu") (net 29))
 (segment (start 121 119.5) (end 109.385 107.885) (width 1.27) (layer "B.Cu") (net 29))
 (segment (start 187.42 101.75) (end 139.25 101.75) (width 1.27) (layer "B.Cu") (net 19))
 (segment (start 208.17 122.5) (end 187.42 101.75) (width 1.27) (layer "B.Cu") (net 19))
 (segment (start 139.25 101.75) (end 136.305 104.695) (width 1.27) (layer "B.Cu") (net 19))
 (segment (start 136.305 104.695) (end 136.305 105.13) (width 1.27) (layer "B.Cu") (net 19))
 (segment (start 208.17 107.75) (end 195.67 95.25) (width 1.27) (layer "B.Cu") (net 21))
 (segment (start 131.225 102.775) (end 131.225 105.13) (width 1.27) (layer "B.Cu") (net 21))
 (segment (start 195.67 95.25) (end 138.75 95.25) (width 1.27) (layer "B.Cu") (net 21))
 (segment (start 138.75 95.25) (end 131.225 102.775) (width 1.27) (layer "B.Cu") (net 21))
 (segment (start 106.845 105.13) (end 106.845 109.595) (width 1.27) (layer "B.Cu") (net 30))
 (segment (start 106.845 109.595) (end 119.29 122.04) (width 1.27) (layer "B.Cu") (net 30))
 (segment (start 119.29 122.04) (end 124.45 122.04) (width 1.27) (layer "B.Cu") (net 30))
 (segment (start 104.305 112.055) (end 104.305 105.13) (width 1.27) (layer "B.Cu") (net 31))
 (segment (start 111.75 119.5) (end 104.305 112.055) (width 1.27) (layer "B.Cu") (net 31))
 (segment (start 105.25 137.5) (end 98.25 137.5) (width 1.27) (layer "B.Cu") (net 37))
 (segment (start 110.55 132.2) (end 105.25 137.5) (width 1.27) (layer "B.Cu") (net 37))
 (segment (start 111.75 132.2) (end 110.55 132.2) (width 1.27) (layer "B.Cu") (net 37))
 (segment (start 178 140) (end 181 137) (width 1.27) (layer "B.Cu") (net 1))
 (segment (start 181 137) (end 181 136.5) (width 1.27) (layer "B.Cu") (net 1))
 (segment (start 182 124.75) (end 182 119.25) (width 1.27) (layer "B.Cu") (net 1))
 (segment (start 181.25 136.25) (end 181.25 125.5) (width 1.27) (layer "B.Cu") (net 1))
 (segment (start 181.25 125.5) (end 182 124.75) (width 1.27) (layer "B.Cu") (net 1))
 (segment (start 114.47 140) (end 178 140) (width 1.27) (layer "B.Cu") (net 1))
 (segment (start 181 136.5) (end 181.25 136.25) (width 1.27) (layer "B.Cu") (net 1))
 (segment (start 111.75 137.28) (end 114.47 140) (width 1.27) (layer "B.Cu") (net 1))
 (segment (start 184 143.5) (end 186 141.5) (width 1.27) (layer "B.Cu") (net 2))
 (segment (start 185.5 124.75) (end 185.5 119.25) (width 1.27) (layer "B.Cu") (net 2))
 (segment (start 186 136) (end 186 125.25) (width 1.27) (layer "B.Cu") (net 2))
 (segment (start 186.25 136.25) (end 186 136) (width 1.27) (layer "B.Cu") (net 2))
 (segment (start 186 141.5) (end 186 136.5) (width 1.27) (layer "B.Cu") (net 2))
 (segment (start 111.75 134.74) (end 111.693503 134.74) (width 1.27) (layer "B.Cu") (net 2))
 (segment (start 109.75 143.5) (end 184 143.5) (width 1.27) (layer "B.Cu") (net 2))
 (segment (start 107.5 138.933503) (end 107.5 141.25) (width 1.27) (layer "B.Cu") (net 2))
 (segment (start 107.5 141.25) (end 109.75 143.5) (width 1.27) (layer "B.Cu") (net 2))
 (segment (start 186 136.5) (end 186.25 136.25) (width 1.27) (layer "B.Cu") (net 2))
 (segment (start 111.693503 134.74) (end 107.5 138.933503) (width 1.27) (layer "B.Cu") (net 2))
 (segment (start 186 125.25) (end 185.5 124.75) (width 1.27) (layer "B.Cu") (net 2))
 (segment (start 98.25 127.5) (end 111.37 127.5) (width 1.27) (layer "B.Cu") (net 35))
 (segment (start 111.37 127.5) (end 111.75 127.12) (width 1.27) (layer "B.Cu") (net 35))
 (segment (start 100.33 124.58) (end 98.25 122.5) (width 1.27) (layer "B.Cu") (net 34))
 (segment (start 111.75 124.58) (end 100.33 124.58) (width 1.27) (layer "B.Cu") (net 34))
 (segment (start 107 132.5) (end 98.25 132.5) (width 1.27) (layer "B.Cu") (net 36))
 (segment (start 111.75 129.66) (end 109.84 129.66) (width 1.27) (layer "B.Cu") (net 36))
 (segment (start 109.84 129.66) (end 107 132.5) (width 1.27) (layer "B.Cu") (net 36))
 (segment (start 210.21 100.25) (end 210.21 107.25) (width 1.27) (layer "B.Cu") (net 33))
 (segment (start 210.5 115.04) (end 210.5 107.96) (width 1.27) (layer "B.Cu") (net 33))
 (segment (start 210.71 99.75) (end 210.21 100.25) (width 1.27) (layer "B.Cu") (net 33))
 (segment (start 210.71 115.25) (end 210.5 115.04) (width 1.27) (layer "B.Cu") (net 33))
 (segment (start 210.71 99.75) (end 210.21 99.25) (width 1.27) (layer "B.Cu") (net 33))
 (segment (start 210.21 99.25) (end 210.21 96.54) (width 1.27) (layer "B.Cu") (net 33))
 (segment (start 210.5 115.46) (end 210.71 115.25) (width 1.27) (layer "B.Cu") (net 33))
 (segment (start 210.46 122.25) (end 210.46 117.522) (width 1.27) (layer "B.Cu") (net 33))
 (segment (start 210.21 96.54) (end 216 90.75) (width 1.27) (layer "B.Cu") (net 33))
 (segment (start 210.5 117.482) (end 210.5 115.46) (width 1.27) (layer "B.Cu") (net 33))
 (segment (start 210.46 117.522) (end 210.5 117.482) (width 1.27) (layer "B.Cu") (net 33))
 (segment (start 210.21 107.25) (end 210.71 107.75) (width 1.27) (layer "B.Cu") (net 33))
 (segment (start 210.5 107.96) (end 210.71 107.75) (width 1.27) (layer "B.Cu") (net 33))
 (segment (start 210.71 122.5) (end 210.46 122.25) (width 1.27) (layer "B.Cu") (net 33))
 (segment (start 216 90.75) (end 216 81) (width 1.27) (layer "B.Cu") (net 33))
 (segment (start 124 113.75) (end 129 113.75) (width 1.27) (layer "B.Cu") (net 26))
 (segment (start 131.5 127.5) (end 126.8 132.2) (width 1.27) (layer "B.Cu") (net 26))
 (segment (start 126.8 132.2) (end 124.45 132.2) (width 1.27) (layer "B.Cu") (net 26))
 (segment (start 129 113.75) (end 131.5 116.25) (width 1.27) (layer "B.Cu") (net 26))
 (segment (start 131.5 116.25) (end 131.5 127.5) (width 1.27) (layer "B.Cu") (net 26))
 (segment (start 117.005 106.755) (end 124 113.75) (width 1.27) (layer "B.Cu") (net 26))
 (segment (start 117.005 105.13) (end 117.005 106.755) (width 1.27) (layer "B.Cu") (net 26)))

